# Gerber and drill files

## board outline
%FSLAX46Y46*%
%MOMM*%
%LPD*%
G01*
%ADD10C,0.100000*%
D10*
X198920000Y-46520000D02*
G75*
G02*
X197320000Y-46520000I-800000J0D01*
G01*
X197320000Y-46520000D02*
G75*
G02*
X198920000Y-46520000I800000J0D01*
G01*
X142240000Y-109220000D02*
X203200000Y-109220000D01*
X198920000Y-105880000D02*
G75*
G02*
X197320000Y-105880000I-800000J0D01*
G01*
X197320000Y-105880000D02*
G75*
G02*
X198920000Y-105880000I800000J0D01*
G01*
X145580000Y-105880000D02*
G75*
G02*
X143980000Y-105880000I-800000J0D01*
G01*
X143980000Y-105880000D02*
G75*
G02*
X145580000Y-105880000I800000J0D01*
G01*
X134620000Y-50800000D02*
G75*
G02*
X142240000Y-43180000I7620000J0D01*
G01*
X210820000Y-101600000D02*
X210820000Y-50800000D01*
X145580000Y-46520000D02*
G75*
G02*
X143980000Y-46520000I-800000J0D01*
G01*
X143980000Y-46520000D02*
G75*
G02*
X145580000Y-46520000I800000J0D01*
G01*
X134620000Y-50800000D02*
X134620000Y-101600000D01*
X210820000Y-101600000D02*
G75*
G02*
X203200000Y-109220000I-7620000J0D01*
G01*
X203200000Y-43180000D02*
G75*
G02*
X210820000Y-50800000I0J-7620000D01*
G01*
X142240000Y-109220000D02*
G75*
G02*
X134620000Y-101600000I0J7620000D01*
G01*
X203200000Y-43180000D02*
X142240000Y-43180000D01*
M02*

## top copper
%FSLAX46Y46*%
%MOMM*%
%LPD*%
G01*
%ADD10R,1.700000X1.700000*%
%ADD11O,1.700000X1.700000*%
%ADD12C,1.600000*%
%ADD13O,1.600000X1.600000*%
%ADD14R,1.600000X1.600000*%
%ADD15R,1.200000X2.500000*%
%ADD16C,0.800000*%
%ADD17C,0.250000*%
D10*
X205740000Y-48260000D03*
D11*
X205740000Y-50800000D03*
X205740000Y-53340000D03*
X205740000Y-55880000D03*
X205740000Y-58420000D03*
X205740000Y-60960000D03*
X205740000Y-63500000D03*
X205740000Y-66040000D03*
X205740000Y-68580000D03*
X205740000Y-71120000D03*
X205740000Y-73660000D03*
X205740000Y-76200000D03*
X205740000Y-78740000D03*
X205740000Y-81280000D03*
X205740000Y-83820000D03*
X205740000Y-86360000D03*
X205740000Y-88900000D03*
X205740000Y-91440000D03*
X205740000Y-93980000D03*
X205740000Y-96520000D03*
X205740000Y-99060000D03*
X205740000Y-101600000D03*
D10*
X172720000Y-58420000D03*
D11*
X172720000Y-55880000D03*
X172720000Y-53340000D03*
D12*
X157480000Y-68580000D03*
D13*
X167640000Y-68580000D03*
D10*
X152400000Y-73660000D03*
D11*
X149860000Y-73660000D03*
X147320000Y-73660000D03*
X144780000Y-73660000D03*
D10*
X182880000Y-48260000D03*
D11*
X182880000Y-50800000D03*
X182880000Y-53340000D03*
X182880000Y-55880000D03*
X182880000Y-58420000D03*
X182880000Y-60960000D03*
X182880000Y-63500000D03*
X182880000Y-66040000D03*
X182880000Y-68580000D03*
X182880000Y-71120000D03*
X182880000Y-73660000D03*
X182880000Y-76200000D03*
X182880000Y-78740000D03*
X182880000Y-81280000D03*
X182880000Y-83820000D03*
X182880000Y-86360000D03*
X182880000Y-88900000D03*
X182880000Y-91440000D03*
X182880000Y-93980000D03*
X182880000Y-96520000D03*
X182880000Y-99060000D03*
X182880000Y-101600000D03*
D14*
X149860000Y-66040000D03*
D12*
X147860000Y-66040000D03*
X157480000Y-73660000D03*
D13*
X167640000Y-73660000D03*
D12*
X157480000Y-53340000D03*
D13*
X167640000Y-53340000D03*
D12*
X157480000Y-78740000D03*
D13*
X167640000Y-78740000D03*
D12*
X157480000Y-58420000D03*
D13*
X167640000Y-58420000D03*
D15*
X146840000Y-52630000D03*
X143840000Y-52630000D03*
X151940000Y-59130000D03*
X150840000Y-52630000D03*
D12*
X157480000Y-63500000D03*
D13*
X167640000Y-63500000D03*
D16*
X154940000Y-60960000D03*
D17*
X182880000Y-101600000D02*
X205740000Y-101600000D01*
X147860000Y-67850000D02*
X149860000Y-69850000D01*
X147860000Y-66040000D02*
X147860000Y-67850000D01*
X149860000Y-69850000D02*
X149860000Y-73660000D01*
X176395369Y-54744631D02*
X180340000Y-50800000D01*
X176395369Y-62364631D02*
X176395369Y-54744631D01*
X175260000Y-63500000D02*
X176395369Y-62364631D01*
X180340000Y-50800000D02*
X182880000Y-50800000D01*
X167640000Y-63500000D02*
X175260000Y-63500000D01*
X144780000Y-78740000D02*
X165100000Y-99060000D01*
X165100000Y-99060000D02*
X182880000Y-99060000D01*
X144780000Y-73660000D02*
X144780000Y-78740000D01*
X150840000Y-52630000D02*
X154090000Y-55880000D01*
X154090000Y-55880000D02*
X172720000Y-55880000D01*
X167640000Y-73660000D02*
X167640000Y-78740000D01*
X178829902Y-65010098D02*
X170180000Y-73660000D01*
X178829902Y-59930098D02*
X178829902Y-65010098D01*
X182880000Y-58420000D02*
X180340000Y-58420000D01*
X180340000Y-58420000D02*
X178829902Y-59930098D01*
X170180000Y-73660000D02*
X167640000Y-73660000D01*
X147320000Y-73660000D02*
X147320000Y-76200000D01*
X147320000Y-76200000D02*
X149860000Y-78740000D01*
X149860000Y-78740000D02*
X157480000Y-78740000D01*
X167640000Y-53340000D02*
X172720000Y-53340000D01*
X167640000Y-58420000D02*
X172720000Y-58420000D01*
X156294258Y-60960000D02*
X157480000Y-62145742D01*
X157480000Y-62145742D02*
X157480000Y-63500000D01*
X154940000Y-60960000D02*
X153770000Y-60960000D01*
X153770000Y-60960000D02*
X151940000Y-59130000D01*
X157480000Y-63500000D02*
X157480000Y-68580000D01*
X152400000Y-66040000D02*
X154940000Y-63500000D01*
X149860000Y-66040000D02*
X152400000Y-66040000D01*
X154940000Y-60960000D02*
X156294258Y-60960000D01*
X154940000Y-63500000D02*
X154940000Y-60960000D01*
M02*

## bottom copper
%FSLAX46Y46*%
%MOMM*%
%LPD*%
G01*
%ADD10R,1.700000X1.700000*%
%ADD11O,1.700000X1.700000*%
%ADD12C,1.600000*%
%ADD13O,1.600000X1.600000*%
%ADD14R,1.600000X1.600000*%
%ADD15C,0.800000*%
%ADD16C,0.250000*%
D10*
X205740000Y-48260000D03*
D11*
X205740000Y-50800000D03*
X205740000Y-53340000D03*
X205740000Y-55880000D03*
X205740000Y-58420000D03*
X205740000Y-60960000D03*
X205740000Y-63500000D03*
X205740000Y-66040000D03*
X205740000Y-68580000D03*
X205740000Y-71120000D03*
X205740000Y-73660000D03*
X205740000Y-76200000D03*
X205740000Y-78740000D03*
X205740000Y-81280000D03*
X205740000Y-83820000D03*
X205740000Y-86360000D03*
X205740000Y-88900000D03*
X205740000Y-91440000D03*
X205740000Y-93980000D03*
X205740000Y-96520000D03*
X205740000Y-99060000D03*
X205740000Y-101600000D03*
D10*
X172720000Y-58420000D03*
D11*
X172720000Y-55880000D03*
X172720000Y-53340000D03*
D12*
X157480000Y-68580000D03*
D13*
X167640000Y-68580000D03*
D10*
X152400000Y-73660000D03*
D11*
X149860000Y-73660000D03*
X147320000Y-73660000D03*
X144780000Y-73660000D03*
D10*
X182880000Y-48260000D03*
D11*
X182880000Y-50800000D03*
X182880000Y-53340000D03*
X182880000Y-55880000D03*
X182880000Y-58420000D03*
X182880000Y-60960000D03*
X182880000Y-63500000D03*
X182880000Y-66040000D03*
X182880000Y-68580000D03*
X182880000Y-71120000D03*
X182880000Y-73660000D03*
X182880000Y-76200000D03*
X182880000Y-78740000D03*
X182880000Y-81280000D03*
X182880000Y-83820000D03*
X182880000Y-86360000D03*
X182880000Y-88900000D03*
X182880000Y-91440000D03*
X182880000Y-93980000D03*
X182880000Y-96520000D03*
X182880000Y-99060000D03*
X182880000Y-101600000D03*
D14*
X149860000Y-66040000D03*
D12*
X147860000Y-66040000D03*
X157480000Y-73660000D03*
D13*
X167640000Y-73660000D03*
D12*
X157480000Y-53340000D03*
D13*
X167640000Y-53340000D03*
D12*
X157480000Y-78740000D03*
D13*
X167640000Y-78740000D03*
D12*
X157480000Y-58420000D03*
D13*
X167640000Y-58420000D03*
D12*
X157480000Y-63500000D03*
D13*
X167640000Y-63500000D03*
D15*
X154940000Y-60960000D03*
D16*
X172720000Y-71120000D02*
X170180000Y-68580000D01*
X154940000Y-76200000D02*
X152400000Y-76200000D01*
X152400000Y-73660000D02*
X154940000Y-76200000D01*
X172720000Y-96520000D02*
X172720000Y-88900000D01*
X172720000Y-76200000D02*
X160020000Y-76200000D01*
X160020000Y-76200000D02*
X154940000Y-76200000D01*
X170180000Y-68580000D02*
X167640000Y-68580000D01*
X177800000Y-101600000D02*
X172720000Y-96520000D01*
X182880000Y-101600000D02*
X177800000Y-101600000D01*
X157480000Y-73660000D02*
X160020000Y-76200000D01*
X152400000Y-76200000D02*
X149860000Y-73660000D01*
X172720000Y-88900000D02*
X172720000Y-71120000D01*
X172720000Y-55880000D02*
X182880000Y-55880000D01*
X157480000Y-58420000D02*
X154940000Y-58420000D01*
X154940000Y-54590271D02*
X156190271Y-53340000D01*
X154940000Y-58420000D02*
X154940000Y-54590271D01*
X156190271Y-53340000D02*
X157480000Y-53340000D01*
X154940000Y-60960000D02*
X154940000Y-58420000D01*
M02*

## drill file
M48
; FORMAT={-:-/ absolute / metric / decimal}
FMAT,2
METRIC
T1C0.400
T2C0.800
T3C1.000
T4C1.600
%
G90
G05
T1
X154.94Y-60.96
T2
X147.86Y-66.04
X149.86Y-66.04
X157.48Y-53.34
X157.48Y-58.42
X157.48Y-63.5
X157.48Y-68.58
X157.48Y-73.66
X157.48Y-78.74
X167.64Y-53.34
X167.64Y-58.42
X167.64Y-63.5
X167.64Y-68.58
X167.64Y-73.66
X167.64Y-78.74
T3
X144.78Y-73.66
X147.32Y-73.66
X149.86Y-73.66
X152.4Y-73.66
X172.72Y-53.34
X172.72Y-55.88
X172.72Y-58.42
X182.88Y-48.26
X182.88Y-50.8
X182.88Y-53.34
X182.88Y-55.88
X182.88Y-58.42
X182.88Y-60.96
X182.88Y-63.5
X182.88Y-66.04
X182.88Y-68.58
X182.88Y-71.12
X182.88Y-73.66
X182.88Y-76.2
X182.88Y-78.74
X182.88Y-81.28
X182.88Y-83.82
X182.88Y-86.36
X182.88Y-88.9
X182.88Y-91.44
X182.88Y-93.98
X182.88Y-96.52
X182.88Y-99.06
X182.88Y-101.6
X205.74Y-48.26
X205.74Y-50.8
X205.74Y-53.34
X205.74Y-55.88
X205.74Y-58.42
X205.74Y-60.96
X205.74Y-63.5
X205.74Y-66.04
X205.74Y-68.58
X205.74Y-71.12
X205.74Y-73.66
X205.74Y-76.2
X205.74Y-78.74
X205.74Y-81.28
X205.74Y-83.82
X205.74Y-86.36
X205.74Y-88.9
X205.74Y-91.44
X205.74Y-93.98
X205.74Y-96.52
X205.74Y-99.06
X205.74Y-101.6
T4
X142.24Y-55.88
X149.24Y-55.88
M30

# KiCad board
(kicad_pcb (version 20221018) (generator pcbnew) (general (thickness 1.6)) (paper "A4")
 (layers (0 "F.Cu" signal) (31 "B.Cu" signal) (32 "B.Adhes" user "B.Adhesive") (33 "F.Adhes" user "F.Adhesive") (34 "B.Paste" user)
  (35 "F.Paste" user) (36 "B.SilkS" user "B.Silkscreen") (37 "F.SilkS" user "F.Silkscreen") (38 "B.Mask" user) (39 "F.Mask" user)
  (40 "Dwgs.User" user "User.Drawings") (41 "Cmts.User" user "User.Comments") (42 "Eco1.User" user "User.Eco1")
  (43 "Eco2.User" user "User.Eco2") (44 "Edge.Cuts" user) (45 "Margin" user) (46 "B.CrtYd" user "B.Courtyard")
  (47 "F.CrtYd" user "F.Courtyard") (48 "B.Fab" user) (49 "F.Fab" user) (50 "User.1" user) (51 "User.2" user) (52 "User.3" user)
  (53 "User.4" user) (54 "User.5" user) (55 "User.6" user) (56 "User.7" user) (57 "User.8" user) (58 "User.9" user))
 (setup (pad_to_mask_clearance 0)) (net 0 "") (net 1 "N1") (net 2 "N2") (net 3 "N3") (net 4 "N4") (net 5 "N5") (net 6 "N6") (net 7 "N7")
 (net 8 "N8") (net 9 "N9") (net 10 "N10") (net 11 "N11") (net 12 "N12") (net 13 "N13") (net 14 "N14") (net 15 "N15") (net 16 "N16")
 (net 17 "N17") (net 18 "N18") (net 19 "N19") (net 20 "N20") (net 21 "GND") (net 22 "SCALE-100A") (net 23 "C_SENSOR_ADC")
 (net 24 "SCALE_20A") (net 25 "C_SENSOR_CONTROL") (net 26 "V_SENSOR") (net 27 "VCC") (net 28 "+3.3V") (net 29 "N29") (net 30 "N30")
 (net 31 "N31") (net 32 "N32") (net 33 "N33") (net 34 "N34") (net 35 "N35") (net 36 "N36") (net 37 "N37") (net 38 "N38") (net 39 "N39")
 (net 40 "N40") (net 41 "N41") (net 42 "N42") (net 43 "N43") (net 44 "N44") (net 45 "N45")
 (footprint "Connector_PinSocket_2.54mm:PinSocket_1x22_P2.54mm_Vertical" (layer "F.Cu") (at 205.74 48.26)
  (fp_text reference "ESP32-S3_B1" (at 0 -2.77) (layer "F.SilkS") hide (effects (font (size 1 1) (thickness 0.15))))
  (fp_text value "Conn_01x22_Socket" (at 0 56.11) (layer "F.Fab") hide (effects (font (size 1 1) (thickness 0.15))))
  (pad "1" thru_hole rect (at 0 0) (size 1.7 1.7) (drill 1) (layers "*.Cu" "*.Mask") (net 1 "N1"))
  (pad "2" thru_hole oval (at 0 2.54) (size 1.7 1.7) (drill 1) (layers "*.Cu" "*.Mask") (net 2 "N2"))
  (pad "3" thru_hole oval (at 0 5.08) (size 1.7 1.7) (drill 1) (layers "*.Cu" "*.Mask") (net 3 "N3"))
  (pad "4" thru_hole oval (at 0 7.62) (size 1.7 1.7) (drill 1) (layers "*.Cu" "*.Mask") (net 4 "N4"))
  (pad "5" thru_hole oval (at 0 10.16) (size 1.7 1.7) (drill 1) (layers "*.Cu" "*.Mask") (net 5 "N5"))
  (pad "6" thru_hole oval (at 0 12.7) (size 1.7 1.7) (drill 1) (layers "*.Cu" "*.Mask") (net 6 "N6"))
  (pad "7" thru_hole oval (at 0 15.24) (size 1.7 1.7) (drill 1) (layers "*.Cu" "*.Mask") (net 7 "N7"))
  (pad "8" thru_hole oval (at 0 17.78) (size 1.7 1.7) (drill 1) (layers "*.Cu" "*.Mask") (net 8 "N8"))
  (pad "9" thru_hole oval (at 0 20.32) (size 1.7 1.7) (drill 1) (layers "*.Cu" "*.Mask") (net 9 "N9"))
  (pad "10" thru_hole oval (at 0 22.86) (size 1.7 1.7) (drill 1) (layers "*.Cu" "*.Mask") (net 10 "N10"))
  (pad "11" thru_hole oval (at 0 25.4) (size 1.7 1.7) (drill 1) (layers "*.Cu" "*.Mask") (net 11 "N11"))
  (pad "12" thru_hole oval (at 0 27.94) (size 1.7 1.7) (drill 1) (layers "*.Cu" "*.Mask") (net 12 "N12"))
  (pad "13" thru_hole oval (at 0 30.48) (size 1.7 1.7) (drill 1) (layers "*.Cu" "*.Mask") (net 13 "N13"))
  (pad "14" thru_hole oval (at 0 33.02) (size 1.7 1.7) (drill 1) (layers "*.Cu" "*.Mask") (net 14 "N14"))
  (pad "15" thru_hole oval (at 0 35.56) (size 1.7 1.7) (drill 1) (layers "*.Cu" "*.Mask") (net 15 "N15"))
  (pad "16" thru_hole oval (at 0 38.1) (size 1.7 1.7) (drill 1) (layers "*.Cu" "*.Mask") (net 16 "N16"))
  (pad "17" thru_hole oval (at 0 40.64) (size 1.7 1.7) (drill 1) (layers "*.Cu" "*.Mask") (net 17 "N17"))
  (pad "18" thru_hole oval (at 0 43.18) (size 1.7 1.7) (drill 1) (layers "*.Cu" "*.Mask") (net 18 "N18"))
  (pad "19" thru_hole oval (at 0 45.72) (size 1.7 1.7) (drill 1) (layers "*.Cu" "*.Mask") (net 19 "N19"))
  (pad "20" thru_hole oval (at 0 48.26) (size 1.7 1.7) (drill 1) (layers "*.Cu" "*.Mask") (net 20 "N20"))
  (pad "21" thru_hole oval (at 0 50.8) (size 1.7 1.7) (drill 1) (layers "*.Cu" "*.Mask") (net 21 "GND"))
  (pad "22" thru_hole oval (at 0 53.34) (size 1.7 1.7) (drill 1) (layers "*.Cu" "*.Mask") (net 21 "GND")))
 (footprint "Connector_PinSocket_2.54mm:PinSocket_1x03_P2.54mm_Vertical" (layer "F.Cu") (at 172.72 58.42 180)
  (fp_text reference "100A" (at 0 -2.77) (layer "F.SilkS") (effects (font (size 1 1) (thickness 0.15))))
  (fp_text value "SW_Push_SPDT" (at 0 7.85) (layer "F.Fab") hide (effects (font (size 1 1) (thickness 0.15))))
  (pad "1" thru_hole rect (at 0 0 180) (size 1.7 1.7) (drill 1) (layers "*.Cu" "*.Mask") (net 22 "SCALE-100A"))
  (pad "2" thru_hole oval (at 0 2.54 180) (size 1.7 1.7) (drill 1) (layers "*.Cu" "*.Mask") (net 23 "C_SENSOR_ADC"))
  (pad "3" thru_hole oval (at 0 5.08 180) (size 1.7 1.7) (drill 1) (layers "*.Cu" "*.Mask") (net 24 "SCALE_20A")))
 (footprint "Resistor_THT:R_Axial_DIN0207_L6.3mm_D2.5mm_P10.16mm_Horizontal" (layer "F.Cu") (at 157.48 68.58)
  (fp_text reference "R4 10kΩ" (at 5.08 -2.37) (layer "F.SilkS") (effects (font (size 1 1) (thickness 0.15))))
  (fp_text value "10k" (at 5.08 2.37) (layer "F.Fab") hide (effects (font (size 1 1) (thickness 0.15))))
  (pad "1" thru_hole circle (at 0 0) (size 1.6 1.6) (drill 0.8) (layers "*.Cu" "*.Mask") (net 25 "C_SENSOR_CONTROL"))
  (pad "2" thru_hole oval (at 10.16 0) (size 1.6 1.6) (drill 0.8) (layers "*.Cu" "*.Mask") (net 21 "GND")))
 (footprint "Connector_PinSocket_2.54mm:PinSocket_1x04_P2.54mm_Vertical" (layer "F.Cu") (at 152.4 73.66 -90)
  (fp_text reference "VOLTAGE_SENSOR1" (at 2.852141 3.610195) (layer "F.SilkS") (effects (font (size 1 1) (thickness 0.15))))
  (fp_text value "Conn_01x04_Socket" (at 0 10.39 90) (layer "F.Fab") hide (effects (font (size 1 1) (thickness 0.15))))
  (pad "1" thru_hole rect (at 0 0 270) (size 1.7 1.7) (drill 1) (layers "*.Cu" "*.Mask") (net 21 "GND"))
  (pad "2" thru_hole oval (at 0 2.54 270) (size 1.7 1.7) (drill 1) (layers "*.Cu" "*.Mask") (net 21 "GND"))
  (pad "3" thru_hole oval (at 0 5.08 270) (size 1.7 1.7) (drill 1) (layers "*.Cu" "*.Mask") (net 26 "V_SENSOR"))
  (pad "4" thru_hole oval (at 0 7.62 270) (size 1.7 1.7) (drill 1) (layers "*.Cu" "*.Mask") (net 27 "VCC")))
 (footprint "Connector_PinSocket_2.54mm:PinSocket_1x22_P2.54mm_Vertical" (layer "F.Cu") (at 182.88 48.26)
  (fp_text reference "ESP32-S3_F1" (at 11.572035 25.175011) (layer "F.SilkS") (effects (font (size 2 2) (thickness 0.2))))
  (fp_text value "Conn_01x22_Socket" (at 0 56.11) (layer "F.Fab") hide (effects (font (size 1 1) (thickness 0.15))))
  (pad "1" thru_hole rect (at 0 0) (size 1.7 1.7) (drill 1) (layers "*.Cu" "*.Mask") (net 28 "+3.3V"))
  (pad "2" thru_hole oval (at 0 2.54) (size 1.7 1.7) (drill 1) (layers "*.Cu" "*.Mask") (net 28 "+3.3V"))
  (pad "3" thru_hole oval (at 0 5.08) (size 1.7 1.7) (drill 1) (layers "*.Cu" "*.Mask") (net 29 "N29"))
  (pad "4" thru_hole oval (at 0 7.62) (size 1.7 1.7) (drill 1) (layers "*.Cu" "*.Mask") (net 23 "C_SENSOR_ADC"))
  (pad "5" thru_hole oval (at 0 10.16) (size 1.7 1.7) (drill 1) (layers "*.Cu" "*.Mask") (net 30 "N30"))
  (pad "6" thru_hole oval (at 0 12.7) (size 1.7 1.7) (drill 1) (layers "*.Cu" "*.Mask") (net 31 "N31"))
  (pad "7" thru_hole oval (at 0 15.24) (size 1.7 1.7) (drill 1) (layers "*.Cu" "*.Mask") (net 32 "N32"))
  (pad "8" thru_hole oval (at 0 17.78) (size 1.7 1.7) (drill 1) (layers "*.Cu" "*.Mask") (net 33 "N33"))
  (pad "9" thru_hole oval (at 0 20.32) (size 1.7 1.7) (drill 1) (layers "*.Cu" "*.Mask") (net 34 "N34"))
  (pad "10" thru_hole oval (at 0 22.86) (size 1.7 1.7) (drill 1) (layers "*.Cu" "*.Mask") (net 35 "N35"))
  (pad "11" thru_hole oval (at 0 25.4) (size 1.7 1.7) (drill 1) (layers "*.Cu" "*.Mask") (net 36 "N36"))
  (pad "12" thru_hole oval (at 0 27.94) (size 1.7 1.7) (drill 1) (layers "*.Cu" "*.Mask") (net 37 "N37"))
  (pad "13" thru_hole oval (at 0 30.48) (size 1.7 1.7) (drill 1) (layers "*.Cu" "*.Mask") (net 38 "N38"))
  (pad "14" thru_hole oval (at 0 33.02) (size 1.7 1.7) (drill 1) (layers "*.Cu" "*.Mask") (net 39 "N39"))
  (pad "15" thru_hole oval (at 0 35.56) (size 1.7 1.7) (drill 1) (layers "*.Cu" "*.Mask") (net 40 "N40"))
  (pad "16" thru_hole oval (at 0 38.1) (size 1.7 1.7) (drill 1) (layers "*.Cu" "*.Mask") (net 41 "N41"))
  (pad "17" thru_hole oval (at 0 40.64) (size 1.7 1.7) (drill 1) (layers "*.Cu" "*.Mask") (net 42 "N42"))
  (pad "18" thru_hole oval (at 0 43.18) (size 1.7 1.7) (drill 1) (layers "*.Cu" "*.Mask") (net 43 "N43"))
  (pad "19" thru_hole oval (at 0 45.72) (size 1.7 1.7) (drill 1) (layers "*.Cu" "*.Mask") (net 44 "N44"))
  (pad "20" thru_hole oval (at 0 48.26) (size 1.7 1.7) (drill 1) (layers "*.Cu" "*.Mask") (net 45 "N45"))
  (pad "21" thru_hole oval (at 0 50.8) (size 1.7 1.7) (drill 1) (layers "*.Cu" "*.Mask") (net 27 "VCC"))
  (pad "22" thru_hole oval (at 0 53.34) (size 1.7 1.7) (drill 1) (layers "*.Cu" "*.Mask") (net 21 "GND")))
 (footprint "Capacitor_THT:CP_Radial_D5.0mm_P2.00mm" (layer "F.Cu") (at 149.86 66.04 180)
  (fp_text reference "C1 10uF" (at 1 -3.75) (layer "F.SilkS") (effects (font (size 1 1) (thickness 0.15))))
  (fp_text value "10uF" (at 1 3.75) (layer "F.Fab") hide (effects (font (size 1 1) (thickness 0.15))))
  (pad "1" thru_hole rect (at 0 0 180) (size 1.6 1.6) (drill 0.8) (layers "*.Cu" "*.Mask") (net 25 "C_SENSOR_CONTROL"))
  (pad "2" thru_hole circle (at 2 0 180) (size 1.6 1.6) (drill 0.8) (layers "*.Cu" "*.Mask") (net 21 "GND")))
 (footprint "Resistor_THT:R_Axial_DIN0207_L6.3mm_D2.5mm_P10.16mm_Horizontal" (layer "F.Cu") (at 157.48 73.66)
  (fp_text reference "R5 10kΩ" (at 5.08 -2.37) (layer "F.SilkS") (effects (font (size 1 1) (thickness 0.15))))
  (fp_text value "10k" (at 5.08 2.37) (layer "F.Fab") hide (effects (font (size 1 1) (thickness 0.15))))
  (pad "1" thru_hole circle (at 0 0) (size 1.6 1.6) (drill 0.8) (layers "*.Cu" "*.Mask") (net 21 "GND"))
  (pad "2" thru_hole oval (at 10.16 0) (size 1.6 1.6) (drill 0.8) (layers "*.Cu" "*.Mask") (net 30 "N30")))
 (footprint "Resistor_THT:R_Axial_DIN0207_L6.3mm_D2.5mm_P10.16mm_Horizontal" (layer "F.Cu") (at 157.48 53.34)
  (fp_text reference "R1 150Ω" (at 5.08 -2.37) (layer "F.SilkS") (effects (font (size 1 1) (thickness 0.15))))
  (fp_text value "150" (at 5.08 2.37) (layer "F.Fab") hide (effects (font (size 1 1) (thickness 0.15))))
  (pad "1" thru_hole circle (at 0 0) (size 1.6 1.6) (drill 0.8) (layers "*.Cu" "*.Mask") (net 25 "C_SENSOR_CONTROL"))
  (pad "2" thru_hole oval (at 10.16 0) (size 1.6 1.6) (drill 0.8) (layers "*.Cu" "*.Mask") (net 24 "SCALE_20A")))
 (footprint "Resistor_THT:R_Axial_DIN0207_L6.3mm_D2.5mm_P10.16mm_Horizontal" (layer "F.Cu") (at 157.48 78.74)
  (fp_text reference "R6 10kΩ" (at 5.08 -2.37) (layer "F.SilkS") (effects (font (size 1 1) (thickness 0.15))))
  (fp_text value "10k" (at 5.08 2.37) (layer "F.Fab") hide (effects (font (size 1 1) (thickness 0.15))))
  (pad "1" thru_hole circle (at 0 0) (size 1.6 1.6) (drill 0.8) (layers "*.Cu" "*.Mask") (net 26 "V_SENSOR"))
  (pad "2" thru_hole oval (at 10.16 0) (size 1.6 1.6) (drill 0.8) (layers "*.Cu" "*.Mask") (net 30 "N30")))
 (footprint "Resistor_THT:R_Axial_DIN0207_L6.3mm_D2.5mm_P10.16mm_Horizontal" (layer "F.Cu") (at 157.48 58.42)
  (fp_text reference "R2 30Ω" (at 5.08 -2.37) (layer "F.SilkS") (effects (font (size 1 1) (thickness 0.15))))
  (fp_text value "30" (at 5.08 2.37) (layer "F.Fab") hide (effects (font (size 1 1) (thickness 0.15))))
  (pad "1" thru_hole circle (at 0 0) (size 1.6 1.6) (drill 0.8) (layers "*.Cu" "*.Mask") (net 25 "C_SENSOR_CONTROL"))
  (pad "2" thru_hole oval (at 10.16 0) (size 1.6 1.6) (drill 0.8) (layers "*.Cu" "*.Mask") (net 22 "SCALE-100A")))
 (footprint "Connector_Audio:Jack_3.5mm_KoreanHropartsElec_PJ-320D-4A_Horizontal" (layer "F.Cu") (at 146.99 55.88)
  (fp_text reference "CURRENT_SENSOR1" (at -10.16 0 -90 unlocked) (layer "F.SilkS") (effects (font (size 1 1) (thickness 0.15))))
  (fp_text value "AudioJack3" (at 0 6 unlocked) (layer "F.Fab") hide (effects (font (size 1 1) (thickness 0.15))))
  (pad "" np_thru_hole circle (at -4.75 0) (size 1.6 1.6) (drill 1.6) (layers "F&B.Cu" "*.Mask"))
  (pad "" np_thru_hole circle (at 2.25 0) (size 1.6 1.6) (drill 1.6) (layers "F&B.Cu" "*.Mask"))
  (pad "R1" smd rect (at -0.15 -3.25) (size 1.2 2.5) (layers "F.Cu" "F.Paste" "F.Mask"))
  (pad "R2" smd rect (at -3.15 -3.25) (size 1.2 2.5) (layers "F.Cu" "F.Paste" "F.Mask"))
  (pad "S" smd rect (at 4.95 3.25) (size 1.2 2.5) (layers "F.Cu" "F.Paste" "F.Mask") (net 25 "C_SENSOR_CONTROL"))
  (pad "T" smd rect (at 3.85 -3.25) (size 1.2 2.5) (layers "F.Cu" "F.Paste" "F.Mask") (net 23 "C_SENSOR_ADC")))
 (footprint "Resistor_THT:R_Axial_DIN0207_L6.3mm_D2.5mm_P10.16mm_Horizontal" (layer "F.Cu") (at 157.48 63.5)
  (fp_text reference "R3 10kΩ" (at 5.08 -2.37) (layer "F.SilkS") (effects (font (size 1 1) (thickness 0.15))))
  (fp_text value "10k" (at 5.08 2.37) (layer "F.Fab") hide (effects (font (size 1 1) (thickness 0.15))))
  (pad "1" thru_hole circle (at 0 0) (size 1.6 1.6) (drill 0.8) (layers "*.Cu" "*.Mask") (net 25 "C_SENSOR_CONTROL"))
  (pad "2" thru_hole oval (at 10.16 0) (size 1.6 1.6) (drill 0.8) (layers "*.Cu" "*.Mask") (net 28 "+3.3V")))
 (gr_circle (center 198.12 46.52) (end 198.92 46.52) (stroke (width 0.1) (type default)) (fill none) (layer "Edge.Cuts"))
 (gr_line (start 142.24 109.22) (end 203.2 109.22) (stroke (width 0.1) (type default)) (layer "Edge.Cuts"))
 (gr_circle (center 198.12 105.88) (end 198.92 105.88) (stroke (width 0.1) (type default)) (fill none) (layer "Edge.Cuts"))
 (gr_circle (center 144.78 105.88) (end 145.58 105.88) (stroke (width 0.1) (type default)) (fill none) (layer "Edge.Cuts"))
 (gr_arc (start 134.62 50.8) (mid 136.851846 45.411846) (end 142.24 43.18) (stroke (width 0.1) (type default)) (layer "Edge.Cuts"))
 (gr_line (start 210.82 101.6) (end 210.82 50.8) (stroke (width 0.1) (type default)) (layer "Edge.Cuts"))
 (gr_circle (center 144.78 46.52) (end 145.58 46.52) (stroke (width 0.1) (type default)) (fill none) (layer "Edge.Cuts"))
 (gr_line (start 134.62 50.8) (end 134.62 101.6) (stroke (width 0.1) (type default)) (layer "Edge.Cuts"))
 (gr_arc (start 210.82 101.6) (mid 208.588154 106.988154) (end 203.2 109.22) (stroke (width 0.1) (type default)) (layer "Edge.Cuts"))
 (gr_arc (start 203.2 43.18) (mid 208.588154 45.411846) (end 210.82 50.8) (stroke (width 0.1) (type default)) (layer "Edge.Cuts"))
 (gr_arc (start 142.24 109.22) (mid 136.851846 106.988154) (end 134.62 101.6) (stroke (width 0.1) (type default)) (layer "Edge.Cuts"))
 (gr_line (start 203.2 43.18) (end 142.24 43.18) (stroke (width 0.1) (type default)) (layer "Edge.Cuts"))
 (segment (start 182.88 101.6) (end 205.74 101.6) (width 0.25) (layer "F.Cu") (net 21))
 (segment (start 147.86 67.85) (end 149.86 69.85) (width 0.25) (layer "F.Cu") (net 21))
 (segment (start 147.86 66.04) (end 147.86 67.85) (width 0.25) (layer "F.Cu") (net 21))
 (segment (start 149.86 69.85) (end 149.86 73.66) (width 0.25) (layer "F.Cu") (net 21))
 (segment (start 172.72 71.12) (end 170.18 68.58) (width 0.25) (layer "B.Cu") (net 21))
 (segment (start 154.94 76.2) (end 152.4 76.2) (width 0.25) (layer "B.Cu") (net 21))
 (segment (start 152.4 73.66) (end 154.94 76.2) (width 0.25) (layer "B.Cu") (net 21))
 (segment (start 172.72 96.52) (end 172.72 88.9) (width 0.25) (layer "B.Cu") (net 21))
 (segment (start 172.72 76.2) (end 160.02 76.2) (width 0.25) (layer "B.Cu") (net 21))
 (segment (start 160.02 76.2) (end 154.94 76.2) (width 0.25) (layer "B.Cu") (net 21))
 (segment (start 170.18 68.58) (end 167.64 68.58) (width 0.25) (layer "B.Cu") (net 21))
 (segment (start 177.8 101.6) (end 172.72 96.52) (width 0.25) (layer "B.Cu") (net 21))
 (segment (start 182.88 101.6) (end 177.8 101.6) (width 0.25) (layer "B.Cu") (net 21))
 (segment (start 157.48 73.66) (end 160.02 76.2) (width 0.25) (layer "B.Cu") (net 21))
 (segment (start 152.4 76.2) (end 149.86 73.66) (width 0.25) (layer "B.Cu") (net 21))
 (segment (start 172.72 88.9) (end 172.72 71.12) (width 0.25) (layer "B.Cu") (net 21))
 (segment (start 176.395369 54.744631) (end 180.34 50.8) (width 0.25) (layer "F.Cu") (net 28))
 (segment (start 176.395369 62.364631) (end 176.395369 54.744631) (width 0.25) (layer "F.Cu") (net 28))
 (segment (start 175.26 63.5) (end 176.395369 62.364631) (width 0.25) (layer "F.Cu") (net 28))
 (segment (start 180.34 50.8) (end 182.88 50.8) (width 0.25) (layer "F.Cu") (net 28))
 (segment (start 167.64 63.5) (end 175.26 63.5) (width 0.25) (layer "F.Cu") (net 28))
 (segment (start 144.78 78.74) (end 165.1 99.06) (width 0.25) (layer "F.Cu") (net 27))
 (segment (start 165.1 99.06) (end 182.88 99.06) (width 0.25) (layer "F.Cu") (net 27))
 (segment (start 144.78 73.66) (end 144.78 78.74) (width 0.25) (layer "F.Cu") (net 27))
 (segment (start 150.84 52.63) (end 154.09 55.88) (width 0.25) (layer "F.Cu") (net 23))
 (segment (start 154.09 55.88) (end 172.72 55.88) (width 0.25) (layer "F.Cu") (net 23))
 (segment (start 172.72 55.88) (end 182.88 55.88) (width 0.25) (layer "B.Cu") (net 23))
 (segment (start 167.64 73.66) (end 167.64 78.74) (width 0.25) (layer "F.Cu") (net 30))
 (segment (start 178.829902 65.010098) (end 170.18 73.66) (width 0.25) (layer "F.Cu") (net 30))
 (segment (start 178.829902 59.930098) (end 178.829902 65.010098) (width 0.25) (layer "F.Cu") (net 30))
 (segment (start 182.88 58.42) (end 180.34 58.42) (width 0.25) (layer "F.Cu") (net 30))
 (segment (start 180.34 58.42) (end 178.829902 59.930098) (width 0.25) (layer "F.Cu") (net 30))
 (segment (start 170.18 73.66) (end 167.64 73.66) (width 0.25) (layer "F.Cu") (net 30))
 (segment (start 147.32 73.66) (end 147.32 76.2) (width 0.25) (layer "F.Cu") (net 26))
 (segment (start 147.32 76.2) (end 149.86 78.74) (width 0.25) (layer "F.Cu") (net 26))
 (segment (start 149.86 78.74) (end 157.48 78.74) (width 0.25) (layer "F.Cu") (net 26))
 (segment (start 167.64 53.34) (end 172.72 53.34) (width 0.25) (layer "F.Cu") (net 24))
 (segment (start 167.64 58.42) (end 172.72 58.42) (width 0.25) (layer "F.Cu") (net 22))
 (segment (start 156.294258 60.96) (end 157.48 62.145742) (width 0.25) (layer "F.Cu") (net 25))
 (segment (start 157.48 62.145742) (end 157.48 63.5) (width 0.25) (layer "F.Cu") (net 25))
 (segment (start 154.94 60.96) (end 153.77 60.96) (width 0.25) (layer "F.Cu") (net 25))
 (segment (start 153.77 60.96) (end 151.94 59.13) (width 0.25) (layer "F.Cu") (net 25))
 (segment (start 157.48 63.5) (end 157.48 68.58) (width 0.25) (layer "F.Cu") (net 25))
 (segment (start 152.4 66.04) (end 154.94 63.5) (width 0.25) (layer "F.Cu") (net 25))
 (segment (start 149.86 66.04) (end 152.4 66.04) (width 0.25) (layer "F.Cu") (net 25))
 (segment (start 154.94 60.96) (end 156.294258 60.96) (width 0.25) (layer "F.Cu") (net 25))
 (segment (start 154.94 63.5) (end 154.94 60.96) (width 0.25) (layer "F.Cu") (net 25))
 (via (at 154.94 60.96) (size 0.8) (drill 0.4) (layers "F.Cu" "B.Cu") (free) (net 25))
 (segment (start 157.48 58.42) (end 154.94 58.42) (width 0.25) (layer "B.Cu") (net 25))
 (segment (start 154.94 54.590271) (end 156.190271 53.34) (width 0.25) (layer "B.Cu") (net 25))
 (segment (start 154.94 58.42) (end 154.94 54.590271) (width 0.25) (layer "B.Cu") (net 25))
 (segment (start 156.190271 53.34) (end 157.48 53.34) (width 0.25) (layer "B.Cu") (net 25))
 (segment (start 154.94 60.96) (end 154.94 58.42) (width 0.25) (layer "B.Cu") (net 25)))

